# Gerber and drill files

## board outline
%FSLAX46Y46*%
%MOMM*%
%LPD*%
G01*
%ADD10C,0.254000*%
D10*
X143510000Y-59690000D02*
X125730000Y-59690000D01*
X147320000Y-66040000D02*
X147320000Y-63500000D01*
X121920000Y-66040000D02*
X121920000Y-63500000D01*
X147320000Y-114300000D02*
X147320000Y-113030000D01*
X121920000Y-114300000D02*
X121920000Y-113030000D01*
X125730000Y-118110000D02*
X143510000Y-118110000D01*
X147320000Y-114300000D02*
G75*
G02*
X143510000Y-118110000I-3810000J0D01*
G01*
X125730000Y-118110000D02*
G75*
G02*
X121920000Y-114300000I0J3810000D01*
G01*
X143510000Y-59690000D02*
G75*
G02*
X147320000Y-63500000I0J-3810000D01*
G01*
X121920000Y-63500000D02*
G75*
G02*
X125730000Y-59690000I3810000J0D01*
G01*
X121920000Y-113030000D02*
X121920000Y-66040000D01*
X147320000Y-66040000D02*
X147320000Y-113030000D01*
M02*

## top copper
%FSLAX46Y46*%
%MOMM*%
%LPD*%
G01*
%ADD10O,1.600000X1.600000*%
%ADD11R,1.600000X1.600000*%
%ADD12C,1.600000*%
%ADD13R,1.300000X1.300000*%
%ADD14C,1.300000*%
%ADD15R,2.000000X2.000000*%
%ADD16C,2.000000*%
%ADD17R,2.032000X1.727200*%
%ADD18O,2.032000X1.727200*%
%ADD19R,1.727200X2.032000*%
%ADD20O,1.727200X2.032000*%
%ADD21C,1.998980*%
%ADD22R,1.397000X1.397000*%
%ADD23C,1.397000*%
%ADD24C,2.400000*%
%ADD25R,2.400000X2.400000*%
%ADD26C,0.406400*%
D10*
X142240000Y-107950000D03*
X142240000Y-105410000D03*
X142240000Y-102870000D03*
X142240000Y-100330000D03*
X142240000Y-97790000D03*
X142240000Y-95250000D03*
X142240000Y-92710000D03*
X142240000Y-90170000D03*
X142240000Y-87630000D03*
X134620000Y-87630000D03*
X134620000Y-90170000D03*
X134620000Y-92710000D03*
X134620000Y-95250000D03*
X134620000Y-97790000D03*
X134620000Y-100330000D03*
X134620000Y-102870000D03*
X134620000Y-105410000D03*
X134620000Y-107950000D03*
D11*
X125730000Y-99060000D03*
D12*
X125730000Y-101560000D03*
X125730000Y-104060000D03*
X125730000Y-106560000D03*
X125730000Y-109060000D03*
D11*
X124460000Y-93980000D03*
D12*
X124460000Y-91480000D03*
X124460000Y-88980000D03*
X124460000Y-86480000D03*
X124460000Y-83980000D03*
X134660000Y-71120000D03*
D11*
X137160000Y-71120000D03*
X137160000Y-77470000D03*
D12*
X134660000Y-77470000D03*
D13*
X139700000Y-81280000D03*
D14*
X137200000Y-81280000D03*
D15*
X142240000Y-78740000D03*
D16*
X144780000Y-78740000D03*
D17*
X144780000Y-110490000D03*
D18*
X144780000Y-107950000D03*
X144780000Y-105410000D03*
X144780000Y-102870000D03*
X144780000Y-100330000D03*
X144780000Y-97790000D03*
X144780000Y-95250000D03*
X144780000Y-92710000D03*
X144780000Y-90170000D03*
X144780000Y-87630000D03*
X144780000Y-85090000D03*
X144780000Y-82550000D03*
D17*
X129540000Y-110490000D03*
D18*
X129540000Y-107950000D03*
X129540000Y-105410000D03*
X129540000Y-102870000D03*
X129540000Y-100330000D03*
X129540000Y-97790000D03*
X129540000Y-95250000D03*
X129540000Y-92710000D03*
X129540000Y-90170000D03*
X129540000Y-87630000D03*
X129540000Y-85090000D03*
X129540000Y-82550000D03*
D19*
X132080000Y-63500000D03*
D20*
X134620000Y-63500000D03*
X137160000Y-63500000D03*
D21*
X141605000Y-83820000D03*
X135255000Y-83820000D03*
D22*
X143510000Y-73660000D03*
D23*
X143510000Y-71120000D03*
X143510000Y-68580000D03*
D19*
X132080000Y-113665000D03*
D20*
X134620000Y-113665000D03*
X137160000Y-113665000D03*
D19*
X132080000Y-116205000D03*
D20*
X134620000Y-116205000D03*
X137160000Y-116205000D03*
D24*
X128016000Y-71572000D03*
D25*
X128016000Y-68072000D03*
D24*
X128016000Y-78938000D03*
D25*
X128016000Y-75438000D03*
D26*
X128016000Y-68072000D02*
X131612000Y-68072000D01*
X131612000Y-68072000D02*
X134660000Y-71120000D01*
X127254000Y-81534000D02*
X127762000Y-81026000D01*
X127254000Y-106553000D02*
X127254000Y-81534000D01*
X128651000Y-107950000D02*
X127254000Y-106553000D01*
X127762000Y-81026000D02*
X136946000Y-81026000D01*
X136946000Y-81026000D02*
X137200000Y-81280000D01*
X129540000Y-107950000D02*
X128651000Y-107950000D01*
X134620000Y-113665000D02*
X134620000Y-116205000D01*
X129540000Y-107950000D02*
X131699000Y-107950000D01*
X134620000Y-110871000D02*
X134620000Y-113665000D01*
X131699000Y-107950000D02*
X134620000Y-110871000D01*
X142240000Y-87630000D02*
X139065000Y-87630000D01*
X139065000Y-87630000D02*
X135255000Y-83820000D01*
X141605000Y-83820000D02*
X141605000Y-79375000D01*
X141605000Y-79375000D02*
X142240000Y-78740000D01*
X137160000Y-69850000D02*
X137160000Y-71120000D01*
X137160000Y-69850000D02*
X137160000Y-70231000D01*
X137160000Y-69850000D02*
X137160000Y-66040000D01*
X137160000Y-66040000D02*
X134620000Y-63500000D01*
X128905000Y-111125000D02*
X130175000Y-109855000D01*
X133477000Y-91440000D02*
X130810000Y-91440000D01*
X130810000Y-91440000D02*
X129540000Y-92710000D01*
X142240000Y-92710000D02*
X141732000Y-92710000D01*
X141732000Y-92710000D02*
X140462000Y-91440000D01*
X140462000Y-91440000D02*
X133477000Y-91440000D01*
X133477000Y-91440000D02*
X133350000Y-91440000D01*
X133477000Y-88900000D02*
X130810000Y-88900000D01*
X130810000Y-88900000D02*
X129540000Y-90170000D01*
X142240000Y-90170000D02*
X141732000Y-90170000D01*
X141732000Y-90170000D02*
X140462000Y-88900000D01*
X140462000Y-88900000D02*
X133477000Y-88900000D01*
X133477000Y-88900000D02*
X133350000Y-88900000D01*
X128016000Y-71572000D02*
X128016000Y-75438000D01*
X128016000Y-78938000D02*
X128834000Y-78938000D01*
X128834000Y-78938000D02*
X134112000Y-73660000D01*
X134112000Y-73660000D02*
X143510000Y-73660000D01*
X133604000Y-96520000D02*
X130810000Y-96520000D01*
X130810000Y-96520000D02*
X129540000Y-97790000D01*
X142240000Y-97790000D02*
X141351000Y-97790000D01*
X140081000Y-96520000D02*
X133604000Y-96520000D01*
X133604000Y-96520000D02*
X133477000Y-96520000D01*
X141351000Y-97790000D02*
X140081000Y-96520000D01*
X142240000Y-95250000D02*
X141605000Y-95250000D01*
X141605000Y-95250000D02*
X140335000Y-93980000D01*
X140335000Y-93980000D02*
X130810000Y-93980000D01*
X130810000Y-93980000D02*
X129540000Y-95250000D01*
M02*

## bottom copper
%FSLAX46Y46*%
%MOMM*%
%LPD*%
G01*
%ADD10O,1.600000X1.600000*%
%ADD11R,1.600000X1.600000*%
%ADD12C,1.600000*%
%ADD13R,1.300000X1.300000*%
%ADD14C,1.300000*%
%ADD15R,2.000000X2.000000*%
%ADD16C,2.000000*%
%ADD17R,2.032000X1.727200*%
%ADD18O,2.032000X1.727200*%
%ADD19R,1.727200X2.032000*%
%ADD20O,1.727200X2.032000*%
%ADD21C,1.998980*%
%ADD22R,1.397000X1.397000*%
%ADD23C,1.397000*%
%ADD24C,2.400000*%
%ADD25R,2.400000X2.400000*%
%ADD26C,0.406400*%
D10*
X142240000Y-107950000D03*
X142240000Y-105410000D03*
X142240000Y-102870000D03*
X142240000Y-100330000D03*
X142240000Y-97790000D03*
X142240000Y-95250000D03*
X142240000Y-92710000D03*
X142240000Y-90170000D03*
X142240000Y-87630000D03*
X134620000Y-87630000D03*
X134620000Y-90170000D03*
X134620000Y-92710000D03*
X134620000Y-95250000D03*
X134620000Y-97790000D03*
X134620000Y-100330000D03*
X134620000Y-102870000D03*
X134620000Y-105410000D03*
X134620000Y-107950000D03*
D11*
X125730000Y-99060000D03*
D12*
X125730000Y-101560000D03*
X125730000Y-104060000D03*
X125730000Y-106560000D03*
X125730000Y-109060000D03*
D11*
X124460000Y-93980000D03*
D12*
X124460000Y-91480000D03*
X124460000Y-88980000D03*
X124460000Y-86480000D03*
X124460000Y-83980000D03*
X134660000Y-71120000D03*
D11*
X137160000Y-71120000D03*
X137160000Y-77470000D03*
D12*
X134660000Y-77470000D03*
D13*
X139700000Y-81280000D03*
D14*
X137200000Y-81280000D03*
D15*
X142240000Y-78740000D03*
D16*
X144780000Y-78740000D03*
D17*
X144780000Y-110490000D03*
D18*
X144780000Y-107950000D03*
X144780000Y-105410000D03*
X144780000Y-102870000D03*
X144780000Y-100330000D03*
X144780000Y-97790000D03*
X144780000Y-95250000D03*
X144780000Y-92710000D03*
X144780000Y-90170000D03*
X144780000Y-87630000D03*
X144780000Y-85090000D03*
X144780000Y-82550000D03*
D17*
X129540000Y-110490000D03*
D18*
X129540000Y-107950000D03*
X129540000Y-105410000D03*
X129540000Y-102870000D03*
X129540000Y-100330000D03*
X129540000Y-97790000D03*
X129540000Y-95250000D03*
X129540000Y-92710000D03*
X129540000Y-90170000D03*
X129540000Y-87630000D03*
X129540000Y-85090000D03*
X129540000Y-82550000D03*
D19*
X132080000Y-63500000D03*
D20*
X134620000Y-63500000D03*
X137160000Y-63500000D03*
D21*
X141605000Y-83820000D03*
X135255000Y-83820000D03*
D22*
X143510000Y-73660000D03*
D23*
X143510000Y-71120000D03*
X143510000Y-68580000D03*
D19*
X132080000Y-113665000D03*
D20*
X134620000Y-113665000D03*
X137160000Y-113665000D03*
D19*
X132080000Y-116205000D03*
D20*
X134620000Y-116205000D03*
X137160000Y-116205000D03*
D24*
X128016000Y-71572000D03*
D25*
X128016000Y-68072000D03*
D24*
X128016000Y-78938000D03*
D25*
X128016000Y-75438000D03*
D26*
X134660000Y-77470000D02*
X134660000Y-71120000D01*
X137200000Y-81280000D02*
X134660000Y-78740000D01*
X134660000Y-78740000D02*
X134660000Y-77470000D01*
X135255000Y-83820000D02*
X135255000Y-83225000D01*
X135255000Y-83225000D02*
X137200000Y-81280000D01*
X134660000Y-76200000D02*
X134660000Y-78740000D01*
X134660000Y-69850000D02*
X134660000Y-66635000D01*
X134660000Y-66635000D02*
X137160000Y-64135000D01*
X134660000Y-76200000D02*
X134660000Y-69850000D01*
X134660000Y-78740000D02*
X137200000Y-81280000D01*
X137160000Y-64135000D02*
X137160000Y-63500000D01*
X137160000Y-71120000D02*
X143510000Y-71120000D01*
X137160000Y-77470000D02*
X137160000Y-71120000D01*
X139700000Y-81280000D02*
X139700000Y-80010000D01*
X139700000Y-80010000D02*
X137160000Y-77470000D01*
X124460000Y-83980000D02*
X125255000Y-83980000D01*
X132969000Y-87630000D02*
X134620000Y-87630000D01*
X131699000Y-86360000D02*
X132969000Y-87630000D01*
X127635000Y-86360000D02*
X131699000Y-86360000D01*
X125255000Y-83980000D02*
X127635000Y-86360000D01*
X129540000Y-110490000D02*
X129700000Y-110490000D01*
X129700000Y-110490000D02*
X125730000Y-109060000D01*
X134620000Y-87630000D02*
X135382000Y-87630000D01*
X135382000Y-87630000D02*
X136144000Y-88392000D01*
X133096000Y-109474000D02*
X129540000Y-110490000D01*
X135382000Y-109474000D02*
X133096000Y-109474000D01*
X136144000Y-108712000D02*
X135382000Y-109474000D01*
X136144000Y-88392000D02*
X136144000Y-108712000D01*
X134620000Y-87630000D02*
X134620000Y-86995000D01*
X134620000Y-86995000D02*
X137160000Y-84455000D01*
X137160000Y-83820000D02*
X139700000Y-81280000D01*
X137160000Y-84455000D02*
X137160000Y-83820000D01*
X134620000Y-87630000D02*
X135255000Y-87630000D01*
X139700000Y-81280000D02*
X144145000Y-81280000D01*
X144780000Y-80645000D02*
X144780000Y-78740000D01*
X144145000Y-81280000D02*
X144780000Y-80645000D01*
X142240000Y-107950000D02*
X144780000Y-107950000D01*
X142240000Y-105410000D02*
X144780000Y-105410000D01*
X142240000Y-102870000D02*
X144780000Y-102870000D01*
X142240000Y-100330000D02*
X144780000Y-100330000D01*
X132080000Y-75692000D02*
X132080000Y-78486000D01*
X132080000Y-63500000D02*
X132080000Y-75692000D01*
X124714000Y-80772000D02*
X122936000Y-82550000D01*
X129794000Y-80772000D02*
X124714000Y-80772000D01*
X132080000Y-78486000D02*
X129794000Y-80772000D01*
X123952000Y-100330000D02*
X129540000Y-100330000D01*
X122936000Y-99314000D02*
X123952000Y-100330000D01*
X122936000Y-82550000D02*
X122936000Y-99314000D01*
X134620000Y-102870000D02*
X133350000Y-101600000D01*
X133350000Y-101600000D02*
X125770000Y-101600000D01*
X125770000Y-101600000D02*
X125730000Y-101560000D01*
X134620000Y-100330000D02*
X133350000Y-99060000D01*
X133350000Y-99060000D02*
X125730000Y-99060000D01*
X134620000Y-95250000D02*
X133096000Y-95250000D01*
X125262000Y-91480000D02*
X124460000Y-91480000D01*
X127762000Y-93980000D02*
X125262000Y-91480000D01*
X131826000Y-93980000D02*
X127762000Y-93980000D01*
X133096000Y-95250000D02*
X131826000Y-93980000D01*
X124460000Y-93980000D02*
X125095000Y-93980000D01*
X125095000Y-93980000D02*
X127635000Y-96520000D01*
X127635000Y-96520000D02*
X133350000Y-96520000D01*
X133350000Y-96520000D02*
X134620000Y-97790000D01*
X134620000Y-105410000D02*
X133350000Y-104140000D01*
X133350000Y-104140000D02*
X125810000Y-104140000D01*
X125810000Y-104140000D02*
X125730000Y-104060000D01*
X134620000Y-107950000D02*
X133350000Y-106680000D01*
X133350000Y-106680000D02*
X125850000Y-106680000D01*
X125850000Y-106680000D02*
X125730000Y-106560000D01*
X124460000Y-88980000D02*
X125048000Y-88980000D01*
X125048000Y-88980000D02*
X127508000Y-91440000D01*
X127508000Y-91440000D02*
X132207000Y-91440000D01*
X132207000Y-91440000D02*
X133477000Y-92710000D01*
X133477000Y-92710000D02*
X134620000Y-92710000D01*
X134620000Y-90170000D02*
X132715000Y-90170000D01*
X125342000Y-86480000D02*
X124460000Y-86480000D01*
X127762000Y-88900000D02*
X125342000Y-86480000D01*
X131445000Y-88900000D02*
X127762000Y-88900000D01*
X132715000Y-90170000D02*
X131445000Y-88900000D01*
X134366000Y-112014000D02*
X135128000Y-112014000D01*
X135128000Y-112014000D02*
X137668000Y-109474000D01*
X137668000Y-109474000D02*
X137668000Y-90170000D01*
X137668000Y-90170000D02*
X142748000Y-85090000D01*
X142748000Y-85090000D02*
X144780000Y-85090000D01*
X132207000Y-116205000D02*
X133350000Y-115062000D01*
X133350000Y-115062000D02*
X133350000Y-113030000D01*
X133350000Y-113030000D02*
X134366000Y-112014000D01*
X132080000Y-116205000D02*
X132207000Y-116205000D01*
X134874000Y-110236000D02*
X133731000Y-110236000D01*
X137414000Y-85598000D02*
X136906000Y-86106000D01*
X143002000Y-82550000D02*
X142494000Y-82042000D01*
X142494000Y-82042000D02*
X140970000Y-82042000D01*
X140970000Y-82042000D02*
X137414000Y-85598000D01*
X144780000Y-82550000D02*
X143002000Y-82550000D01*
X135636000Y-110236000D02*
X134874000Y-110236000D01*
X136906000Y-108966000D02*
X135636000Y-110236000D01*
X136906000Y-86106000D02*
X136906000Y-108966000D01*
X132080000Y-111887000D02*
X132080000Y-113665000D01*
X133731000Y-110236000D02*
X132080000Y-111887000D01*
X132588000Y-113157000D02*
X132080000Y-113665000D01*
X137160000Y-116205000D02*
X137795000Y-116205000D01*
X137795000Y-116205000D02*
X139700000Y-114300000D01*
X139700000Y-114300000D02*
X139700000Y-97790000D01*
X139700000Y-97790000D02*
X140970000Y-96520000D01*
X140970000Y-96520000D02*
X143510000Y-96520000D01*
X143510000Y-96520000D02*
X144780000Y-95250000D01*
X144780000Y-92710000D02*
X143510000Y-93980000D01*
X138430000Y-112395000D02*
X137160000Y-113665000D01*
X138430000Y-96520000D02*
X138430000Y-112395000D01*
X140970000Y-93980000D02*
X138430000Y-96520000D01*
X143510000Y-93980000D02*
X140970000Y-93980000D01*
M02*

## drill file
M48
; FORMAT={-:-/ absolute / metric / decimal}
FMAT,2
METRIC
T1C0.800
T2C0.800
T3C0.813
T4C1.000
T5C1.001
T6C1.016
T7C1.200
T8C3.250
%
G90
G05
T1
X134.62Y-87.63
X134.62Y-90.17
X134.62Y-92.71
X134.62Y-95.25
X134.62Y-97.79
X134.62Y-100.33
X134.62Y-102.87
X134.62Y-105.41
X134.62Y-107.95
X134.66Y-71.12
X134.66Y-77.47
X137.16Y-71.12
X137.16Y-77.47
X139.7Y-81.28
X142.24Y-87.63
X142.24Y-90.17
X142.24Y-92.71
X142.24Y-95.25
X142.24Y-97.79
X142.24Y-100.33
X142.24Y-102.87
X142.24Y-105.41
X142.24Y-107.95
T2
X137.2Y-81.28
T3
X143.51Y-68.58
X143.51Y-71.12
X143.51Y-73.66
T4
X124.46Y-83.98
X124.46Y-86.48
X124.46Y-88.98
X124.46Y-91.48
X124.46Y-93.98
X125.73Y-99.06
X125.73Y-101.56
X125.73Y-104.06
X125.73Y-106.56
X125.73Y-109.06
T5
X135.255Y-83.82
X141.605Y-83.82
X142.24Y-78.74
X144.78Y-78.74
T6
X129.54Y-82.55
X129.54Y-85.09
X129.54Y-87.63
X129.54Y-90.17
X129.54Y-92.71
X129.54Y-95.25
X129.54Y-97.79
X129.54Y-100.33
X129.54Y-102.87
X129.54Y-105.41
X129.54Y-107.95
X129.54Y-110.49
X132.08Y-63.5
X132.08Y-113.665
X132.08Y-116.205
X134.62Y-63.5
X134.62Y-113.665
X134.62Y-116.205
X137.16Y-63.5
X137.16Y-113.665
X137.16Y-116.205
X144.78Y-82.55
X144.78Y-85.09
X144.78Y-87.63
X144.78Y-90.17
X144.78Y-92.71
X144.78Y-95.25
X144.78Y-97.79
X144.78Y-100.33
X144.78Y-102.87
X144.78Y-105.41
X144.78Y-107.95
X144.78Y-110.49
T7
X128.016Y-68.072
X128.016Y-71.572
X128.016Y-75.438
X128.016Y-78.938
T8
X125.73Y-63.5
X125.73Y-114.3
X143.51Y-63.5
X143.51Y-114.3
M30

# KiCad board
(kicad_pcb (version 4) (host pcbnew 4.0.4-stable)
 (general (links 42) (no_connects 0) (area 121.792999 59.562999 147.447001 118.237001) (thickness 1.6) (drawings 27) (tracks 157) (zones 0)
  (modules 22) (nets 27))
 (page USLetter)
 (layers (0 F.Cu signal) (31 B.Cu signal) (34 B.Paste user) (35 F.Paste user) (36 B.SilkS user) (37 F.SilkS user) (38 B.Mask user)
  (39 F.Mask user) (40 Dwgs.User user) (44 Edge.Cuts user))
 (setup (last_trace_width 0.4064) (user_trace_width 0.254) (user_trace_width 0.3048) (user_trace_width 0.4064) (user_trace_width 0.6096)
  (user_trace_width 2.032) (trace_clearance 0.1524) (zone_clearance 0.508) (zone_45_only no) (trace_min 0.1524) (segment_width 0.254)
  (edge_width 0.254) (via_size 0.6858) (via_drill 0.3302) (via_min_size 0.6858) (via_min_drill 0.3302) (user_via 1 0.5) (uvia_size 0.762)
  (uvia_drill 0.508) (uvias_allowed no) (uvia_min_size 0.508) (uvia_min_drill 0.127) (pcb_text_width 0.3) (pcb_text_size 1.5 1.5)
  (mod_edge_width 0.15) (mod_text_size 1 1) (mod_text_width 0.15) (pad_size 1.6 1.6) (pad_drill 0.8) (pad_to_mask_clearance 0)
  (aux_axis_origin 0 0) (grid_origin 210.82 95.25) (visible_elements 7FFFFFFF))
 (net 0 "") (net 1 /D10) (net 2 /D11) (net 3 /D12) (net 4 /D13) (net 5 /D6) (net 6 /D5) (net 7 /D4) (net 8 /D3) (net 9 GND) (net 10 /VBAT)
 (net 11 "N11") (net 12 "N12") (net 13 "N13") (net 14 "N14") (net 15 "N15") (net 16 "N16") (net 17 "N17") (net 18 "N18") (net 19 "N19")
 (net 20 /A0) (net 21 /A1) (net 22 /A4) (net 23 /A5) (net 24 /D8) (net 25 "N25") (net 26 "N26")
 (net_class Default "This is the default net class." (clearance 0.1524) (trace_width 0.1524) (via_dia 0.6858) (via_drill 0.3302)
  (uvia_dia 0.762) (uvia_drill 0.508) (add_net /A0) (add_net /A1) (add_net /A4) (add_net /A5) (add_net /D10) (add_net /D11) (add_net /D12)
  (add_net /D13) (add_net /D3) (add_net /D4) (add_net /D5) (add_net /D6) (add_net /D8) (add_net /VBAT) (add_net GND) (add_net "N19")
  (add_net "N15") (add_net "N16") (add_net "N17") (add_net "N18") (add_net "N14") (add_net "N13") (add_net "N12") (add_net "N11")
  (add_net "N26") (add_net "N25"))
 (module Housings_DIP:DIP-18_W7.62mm (layer F.Cu) (at 142.24 107.95 180)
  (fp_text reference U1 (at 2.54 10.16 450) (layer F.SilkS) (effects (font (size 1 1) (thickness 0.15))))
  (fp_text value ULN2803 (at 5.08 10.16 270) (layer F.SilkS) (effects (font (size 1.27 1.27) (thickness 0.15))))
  (pad 1 thru_hole oval (at 0 0 180) (size 1.6 1.6) (drill 0.8) (layers *.Cu *.Mask F.SilkS) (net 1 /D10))
  (pad 2 thru_hole oval (at 0 2.54 180) (size 1.6 1.6) (drill 0.8) (layers *.Cu *.Mask F.SilkS) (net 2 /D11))
  (pad 3 thru_hole oval (at 0 5.08 180) (size 1.6 1.6) (drill 0.8) (layers *.Cu *.Mask F.SilkS) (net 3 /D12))
  (pad 4 thru_hole oval (at 0 7.62 180) (size 1.6 1.6) (drill 0.8) (layers *.Cu *.Mask F.SilkS) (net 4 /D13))
  (pad 5 thru_hole oval (at 0 10.16 180) (size 1.6 1.6) (drill 0.8) (layers *.Cu *.Mask F.SilkS) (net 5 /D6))
  (pad 6 thru_hole oval (at 0 12.7 180) (size 1.6 1.6) (drill 0.8) (layers *.Cu *.Mask F.SilkS) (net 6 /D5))
  (pad 7 thru_hole oval (at 0 15.24 180) (size 1.6 1.6) (drill 0.8) (layers *.Cu *.Mask F.SilkS) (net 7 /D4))
  (pad 8 thru_hole oval (at 0 17.78 180) (size 1.6 1.6) (drill 0.8) (layers *.Cu *.Mask F.SilkS) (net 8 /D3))
  (pad 9 thru_hole oval (at 0 20.32 180) (size 1.6 1.6) (drill 0.8) (layers *.Cu *.Mask F.SilkS) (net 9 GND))
  (pad 10 thru_hole oval (at 7.62 20.32 180) (size 1.6 1.6) (drill 0.8) (layers *.Cu *.Mask F.SilkS) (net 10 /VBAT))
  (pad 11 thru_hole oval (at 7.62 17.78 180) (size 1.6 1.6) (drill 0.8) (layers *.Cu *.Mask F.SilkS) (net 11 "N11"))
  (pad 12 thru_hole oval (at 7.62 15.24 180) (size 1.6 1.6) (drill 0.8) (layers *.Cu *.Mask F.SilkS) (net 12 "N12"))
  (pad 13 thru_hole oval (at 7.62 12.7 180) (size 1.6 1.6) (drill 0.8) (layers *.Cu *.Mask F.SilkS) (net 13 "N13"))
  (pad 14 thru_hole oval (at 7.62 10.16 180) (size 1.6 1.6) (drill 0.8) (layers *.Cu *.Mask F.SilkS) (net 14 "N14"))
  (pad 15 thru_hole oval (at 7.62 7.62 180) (size 1.6 1.6) (drill 0.8) (layers *.Cu *.Mask F.SilkS) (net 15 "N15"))
  (pad 16 thru_hole oval (at 7.62 5.08 180) (size 1.6 1.6) (drill 0.8) (layers *.Cu *.Mask F.SilkS) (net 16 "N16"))
  (pad 17 thru_hole oval (at 7.62 2.54 180) (size 1.6 1.6) (drill 0.8) (layers *.Cu *.Mask F.SilkS) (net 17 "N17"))
  (pad 18 thru_hole oval (at 7.62 0 180) (size 1.6 1.6) (drill 0.8) (layers *.Cu *.Mask F.SilkS) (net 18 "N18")))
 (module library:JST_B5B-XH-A (layer F.Cu) (at 125.73 99.06 270)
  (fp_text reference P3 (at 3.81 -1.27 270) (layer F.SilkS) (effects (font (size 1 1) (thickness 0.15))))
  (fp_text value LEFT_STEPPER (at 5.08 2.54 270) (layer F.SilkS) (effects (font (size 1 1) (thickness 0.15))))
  (pad 1 thru_hole rect (at 0 0 270) (size 1.6 1.6) (drill 1) (layers *.Cu *.Mask F.SilkS) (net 15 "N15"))
  (pad 2 thru_hole circle (at 2.5 0 270) (size 1.6 1.6) (drill 1) (layers *.Cu *.Mask F.SilkS) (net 16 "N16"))
  (pad 3 thru_hole circle (at 5 0 270) (size 1.6 1.6) (drill 1) (layers *.Cu *.Mask F.SilkS) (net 17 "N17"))
  (pad 4 thru_hole circle (at 7.5 0 270) (size 1.6 1.6) (drill 1) (layers *.Cu *.Mask F.SilkS) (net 18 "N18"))
  (pad 5 thru_hole circle (at 10 0 270) (size 1.6 1.6) (drill 1) (layers *.Cu *.Mask F.SilkS) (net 10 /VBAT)))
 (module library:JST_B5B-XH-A (layer F.Cu) (at 124.46 93.98 90)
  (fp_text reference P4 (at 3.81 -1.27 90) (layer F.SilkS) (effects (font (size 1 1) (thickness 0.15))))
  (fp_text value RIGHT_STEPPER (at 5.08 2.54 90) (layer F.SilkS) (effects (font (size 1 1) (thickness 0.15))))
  (pad 1 thru_hole rect (at 0 0 90) (size 1.6 1.6) (drill 1) (layers *.Cu *.Mask F.SilkS) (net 14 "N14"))
  (pad 2 thru_hole circle (at 2.5 0 90) (size 1.6 1.6) (drill 1) (layers *.Cu *.Mask F.SilkS) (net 13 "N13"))
  (pad 3 thru_hole circle (at 5 0 90) (size 1.6 1.6) (drill 1) (layers *.Cu *.Mask F.SilkS) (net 12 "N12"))
  (pad 4 thru_hole circle (at 7.5 0 90) (size 1.6 1.6) (drill 1) (layers *.Cu *.Mask F.SilkS) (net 11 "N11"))
  (pad 5 thru_hole circle (at 10 0 90) (size 1.6 1.6) (drill 1) (layers *.Cu *.Mask F.SilkS) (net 10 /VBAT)))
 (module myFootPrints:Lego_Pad (layer F.Cu) (at 125.73 114.3)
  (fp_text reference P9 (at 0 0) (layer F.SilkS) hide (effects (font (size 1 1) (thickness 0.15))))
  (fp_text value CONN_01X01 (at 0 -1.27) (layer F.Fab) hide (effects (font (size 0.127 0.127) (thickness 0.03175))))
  (pad "" np_thru_hole circle (at 0 0) (size 3.25 3.25) (drill 3.25) (layers *.Cu *.Mask)))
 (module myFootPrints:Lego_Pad (layer F.Cu) (at 143.51 114.3)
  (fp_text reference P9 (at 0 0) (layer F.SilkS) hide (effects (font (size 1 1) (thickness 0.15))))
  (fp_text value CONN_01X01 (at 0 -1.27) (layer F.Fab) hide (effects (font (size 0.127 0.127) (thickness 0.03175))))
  (pad "" np_thru_hole circle (at 0 0) (size 3.25 3.25) (drill 3.25) (layers *.Cu *.Mask)))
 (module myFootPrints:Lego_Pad (layer F.Cu) (at 143.51 63.5)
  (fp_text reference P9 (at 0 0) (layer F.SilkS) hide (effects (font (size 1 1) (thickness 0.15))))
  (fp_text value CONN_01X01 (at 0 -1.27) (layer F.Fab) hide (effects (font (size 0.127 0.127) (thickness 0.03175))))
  (pad "" np_thru_hole circle (at 0 0) (size 3.25 3.25) (drill 3.25) (layers *.Cu *.Mask)))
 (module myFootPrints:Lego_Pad (layer F.Cu) (at 125.73 63.5)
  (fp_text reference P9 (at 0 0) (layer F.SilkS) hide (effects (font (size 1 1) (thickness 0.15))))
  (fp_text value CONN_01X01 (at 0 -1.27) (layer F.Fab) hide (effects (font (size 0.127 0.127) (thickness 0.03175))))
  (pad "" np_thru_hole circle (at 0 0) (size 3.25 3.25) (drill 3.25) (layers *.Cu *.Mask)))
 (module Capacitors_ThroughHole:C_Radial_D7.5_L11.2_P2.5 (layer F.Cu) (at 137.16 71.12 180)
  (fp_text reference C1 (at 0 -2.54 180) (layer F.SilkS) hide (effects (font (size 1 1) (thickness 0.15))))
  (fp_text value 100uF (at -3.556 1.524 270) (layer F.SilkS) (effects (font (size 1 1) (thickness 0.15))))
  (pad 2 thru_hole circle (at 2.5 0 180) (size 1.6 1.6) (drill 0.8) (layers *.Cu *.Mask F.SilkS) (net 9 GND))
  (pad 1 thru_hole rect (at 0 0 180) (size 1.6 1.6) (drill 0.8) (layers *.Cu *.Mask F.SilkS) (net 10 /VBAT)))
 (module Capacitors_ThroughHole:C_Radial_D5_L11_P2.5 (layer F.Cu) (at 137.16 77.47 180)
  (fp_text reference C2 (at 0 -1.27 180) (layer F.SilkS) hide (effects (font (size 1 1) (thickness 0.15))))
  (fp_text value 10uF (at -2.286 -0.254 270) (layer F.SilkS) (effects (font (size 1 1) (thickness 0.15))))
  (pad 1 thru_hole rect (at 0 0 180) (size 1.6 1.6) (drill 0.8) (layers *.Cu *.Mask F.SilkS) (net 10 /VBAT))
  (pad 2 thru_hole circle (at 2.5 0 180) (size 1.6 1.6) (drill 0.8) (layers *.Cu *.Mask F.SilkS) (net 9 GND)))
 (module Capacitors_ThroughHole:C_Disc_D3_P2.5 (layer F.Cu) (at 139.7 81.28 180)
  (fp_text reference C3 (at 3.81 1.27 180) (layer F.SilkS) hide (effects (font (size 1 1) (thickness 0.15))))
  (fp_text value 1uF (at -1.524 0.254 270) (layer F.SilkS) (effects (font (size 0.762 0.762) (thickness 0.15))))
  (pad 1 thru_hole rect (at 0 0 180) (size 1.3 1.3) (drill 0.8) (layers *.Cu *.Mask F.SilkS) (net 10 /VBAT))
  (pad 2 thru_hole circle (at 2.5 0 180) (size 1.3 1.3) (drill 0.8001) (layers *.Cu *.Mask F.SilkS) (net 9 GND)))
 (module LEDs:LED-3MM (layer F.Cu) (at 142.24 78.74)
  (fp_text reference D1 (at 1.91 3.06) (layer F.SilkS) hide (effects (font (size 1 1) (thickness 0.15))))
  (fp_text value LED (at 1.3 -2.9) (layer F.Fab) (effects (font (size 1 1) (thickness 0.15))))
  (pad 1 thru_hole rect (at 0 0 90) (size 2 2) (drill 1.00076) (layers *.Cu *.Mask F.SilkS) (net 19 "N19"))
  (pad 2 thru_hole circle (at 2.54 0) (size 2 2) (drill 1.00076) (layers *.Cu *.Mask F.SilkS) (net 10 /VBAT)))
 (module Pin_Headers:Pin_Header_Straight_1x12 (layer F.Cu) (at 144.78 110.49 180)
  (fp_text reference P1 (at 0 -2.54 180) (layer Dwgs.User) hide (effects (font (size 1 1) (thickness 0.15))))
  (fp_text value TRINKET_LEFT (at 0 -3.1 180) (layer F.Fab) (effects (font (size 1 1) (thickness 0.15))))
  (pad 1 thru_hole rect (at 0 0 180) (size 2.032 1.7272) (drill 1.016) (layers *.Cu *.Mask F.SilkS))
  (pad 2 thru_hole oval (at 0 2.54 180) (size 2.032 1.7272) (drill 1.016) (layers *.Cu *.Mask F.SilkS) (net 1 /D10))
  (pad 3 thru_hole oval (at 0 5.08 180) (size 2.032 1.7272) (drill 1.016) (layers *.Cu *.Mask F.SilkS) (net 2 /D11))
  (pad 4 thru_hole oval (at 0 7.62 180) (size 2.032 1.7272) (drill 1.016) (layers *.Cu *.Mask F.SilkS) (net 3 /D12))
  (pad 5 thru_hole oval (at 0 10.16 180) (size 2.032 1.7272) (drill 1.016) (layers *.Cu *.Mask F.SilkS) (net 4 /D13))
  (pad 6 thru_hole oval (at 0 12.7 180) (size 2.032 1.7272) (drill 1.016) (layers *.Cu *.Mask F.SilkS))
  (pad 7 thru_hole oval (at 0 15.24 180) (size 2.032 1.7272) (drill 1.016) (layers *.Cu *.Mask F.SilkS) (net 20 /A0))
  (pad 8 thru_hole oval (at 0 17.78 180) (size 2.032 1.7272) (drill 1.016) (layers *.Cu *.Mask F.SilkS) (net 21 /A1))
  (pad 9 thru_hole oval (at 0 20.32 180) (size 2.032 1.7272) (drill 1.016) (layers *.Cu *.Mask F.SilkS))
  (pad 10 thru_hole oval (at 0 22.86 180) (size 2.032 1.7272) (drill 1.016) (layers *.Cu *.Mask F.SilkS))
  (pad 11 thru_hole oval (at 0 25.4 180) (size 2.032 1.7272) (drill 1.016) (layers *.Cu *.Mask F.SilkS) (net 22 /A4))
  (pad 12 thru_hole oval (at 0 27.94 180) (size 2.032 1.7272) (drill 1.016) (layers *.Cu *.Mask F.SilkS) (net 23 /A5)))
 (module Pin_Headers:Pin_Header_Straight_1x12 (layer F.Cu) (at 129.54 110.49 180)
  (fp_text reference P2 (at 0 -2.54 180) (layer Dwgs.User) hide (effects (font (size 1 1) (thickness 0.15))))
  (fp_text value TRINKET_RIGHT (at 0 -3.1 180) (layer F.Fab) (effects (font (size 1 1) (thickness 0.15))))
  (pad 1 thru_hole rect (at 0 0 180) (size 2.032 1.7272) (drill 1.016) (layers *.Cu *.Mask F.SilkS) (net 10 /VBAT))
  (pad 2 thru_hole oval (at 0 2.54 180) (size 2.032 1.7272) (drill 1.016) (layers *.Cu *.Mask F.SilkS) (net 9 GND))
  (pad 3 thru_hole oval (at 0 5.08 180) (size 2.032 1.7272) (drill 1.016) (layers *.Cu *.Mask F.SilkS))
  (pad 4 thru_hole oval (at 0 7.62 180) (size 2.032 1.7272) (drill 1.016) (layers *.Cu *.Mask F.SilkS))
  (pad 5 thru_hole oval (at 0 10.16 180) (size 2.032 1.7272) (drill 1.016) (layers *.Cu *.Mask F.SilkS) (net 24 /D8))
  (pad 6 thru_hole oval (at 0 12.7 180) (size 2.032 1.7272) (drill 1.016) (layers *.Cu *.Mask F.SilkS) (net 5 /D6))
  (pad 7 thru_hole oval (at 0 15.24 180) (size 2.032 1.7272) (drill 1.016) (layers *.Cu *.Mask F.SilkS) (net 6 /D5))
  (pad 8 thru_hole oval (at 0 17.78 180) (size 2.032 1.7272) (drill 1.016) (layers *.Cu *.Mask F.SilkS) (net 7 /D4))
  (pad 9 thru_hole oval (at 0 20.32 180) (size 2.032 1.7272) (drill 1.016) (layers *.Cu *.Mask F.SilkS) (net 8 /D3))
  (pad 10 thru_hole oval (at 0 22.86 180) (size 2.032 1.7272) (drill 1.016) (layers *.Cu *.Mask F.SilkS))
  (pad 11 thru_hole oval (at 0 25.4 180) (size 2.032 1.7272) (drill 1.016) (layers *.Cu *.Mask F.SilkS))
  (pad 12 thru_hole oval (at 0 27.94 180) (size 2.032 1.7272) (drill 1.016) (layers *.Cu *.Mask F.SilkS)))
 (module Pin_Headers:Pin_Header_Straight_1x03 (layer F.Cu) (at 132.08 63.5 90)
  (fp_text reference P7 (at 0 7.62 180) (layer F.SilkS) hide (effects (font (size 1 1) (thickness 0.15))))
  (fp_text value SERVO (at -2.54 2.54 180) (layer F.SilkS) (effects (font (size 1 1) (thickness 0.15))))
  (pad 1 thru_hole rect (at 0 0 90) (size 2.032 1.7272) (drill 1.016) (layers *.Cu *.Mask F.SilkS) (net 24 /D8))
  (pad 2 thru_hole oval (at 0 2.54 90) (size 2.032 1.7272) (drill 1.016) (layers *.Cu *.Mask F.SilkS) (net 10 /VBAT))
  (pad 3 thru_hole oval (at 0 5.08 90) (size 2.032 1.7272) (drill 1.016) (layers *.Cu *.Mask F.SilkS) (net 9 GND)))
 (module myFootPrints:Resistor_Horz (layer F.Cu) (at 138.43 83.82 180)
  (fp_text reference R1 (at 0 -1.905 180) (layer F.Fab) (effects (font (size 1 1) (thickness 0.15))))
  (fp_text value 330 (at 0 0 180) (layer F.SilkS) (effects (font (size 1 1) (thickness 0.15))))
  (pad 1 thru_hole circle (at -3.175 0 180) (size 1.99898 1.99898) (drill 1.00076) (layers *.Cu *.SilkS *.Mask) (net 19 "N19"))
  (pad 2 thru_hole circle (at 3.175 0 180) (size 1.99898 1.99898) (drill 1.00076) (layers *.Cu *.SilkS *.Mask) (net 9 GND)))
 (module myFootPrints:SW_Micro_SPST (layer F.Cu) (at 143.51 71.12 90)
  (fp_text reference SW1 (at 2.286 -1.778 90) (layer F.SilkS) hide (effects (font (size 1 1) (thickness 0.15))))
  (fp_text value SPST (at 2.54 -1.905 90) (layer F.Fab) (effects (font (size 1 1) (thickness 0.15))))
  (pad 1 thru_hole rect (at -2.54 0 90) (size 1.397 1.397) (drill 0.8128) (layers *.Cu *.Mask F.SilkS) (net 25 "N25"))
  (pad 2 thru_hole circle (at 0 0 90) (size 1.397 1.397) (drill 0.8128) (layers *.Cu *.Mask F.SilkS) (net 10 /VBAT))
  (pad 3 thru_hole circle (at 2.54 0 90) (size 1.397 1.397) (drill 0.8128) (layers *.Cu *.Mask F.SilkS)))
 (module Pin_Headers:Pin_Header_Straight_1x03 (layer F.Cu) (at 132.08 113.665 90)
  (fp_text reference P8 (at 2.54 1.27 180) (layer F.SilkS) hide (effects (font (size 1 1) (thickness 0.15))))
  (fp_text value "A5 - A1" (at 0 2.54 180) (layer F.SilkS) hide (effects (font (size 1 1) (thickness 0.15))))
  (pad 1 thru_hole rect (at 0 0 90) (size 2.032 1.7272) (drill 1.016) (layers *.Cu *.Mask F.SilkS) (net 23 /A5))
  (pad 2 thru_hole oval (at 0 2.54 90) (size 2.032 1.7272) (drill 1.016) (layers *.Cu *.Mask F.SilkS) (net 9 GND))
  (pad 3 thru_hole oval (at 0 5.08 90) (size 2.032 1.7272) (drill 1.016) (layers *.Cu *.Mask F.SilkS) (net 21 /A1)))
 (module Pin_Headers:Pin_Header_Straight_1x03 (layer F.Cu) (at 132.08 116.205 90)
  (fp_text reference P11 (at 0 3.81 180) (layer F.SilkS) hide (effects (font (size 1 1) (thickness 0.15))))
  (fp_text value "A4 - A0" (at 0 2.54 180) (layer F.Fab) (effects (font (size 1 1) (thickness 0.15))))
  (pad 1 thru_hole rect (at 0 0 90) (size 2.032 1.7272) (drill 1.016) (layers *.Cu *.Mask F.SilkS) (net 22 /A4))
  (pad 2 thru_hole oval (at 0 2.54 90) (size 2.032 1.7272) (drill 1.016) (layers *.Cu *.Mask F.SilkS) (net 9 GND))
  (pad 3 thru_hole oval (at 0 5.08 90) (size 2.032 1.7272) (drill 1.016) (layers *.Cu *.Mask F.SilkS) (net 20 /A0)))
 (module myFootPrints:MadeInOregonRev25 (layer F.Cu) (at 138.43 102.235 90)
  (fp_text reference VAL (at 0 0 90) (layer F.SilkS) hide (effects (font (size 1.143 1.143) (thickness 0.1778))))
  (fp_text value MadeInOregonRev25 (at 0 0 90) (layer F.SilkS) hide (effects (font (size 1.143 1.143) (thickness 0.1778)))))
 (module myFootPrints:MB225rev (layer F.Cu) (at 138.43 109.22 90)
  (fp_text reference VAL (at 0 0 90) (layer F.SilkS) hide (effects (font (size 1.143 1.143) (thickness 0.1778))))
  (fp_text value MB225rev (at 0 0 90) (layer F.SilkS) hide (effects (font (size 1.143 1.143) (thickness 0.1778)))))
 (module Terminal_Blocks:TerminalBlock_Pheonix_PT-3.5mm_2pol (layer F.Cu) (at 128.016 68.072 270)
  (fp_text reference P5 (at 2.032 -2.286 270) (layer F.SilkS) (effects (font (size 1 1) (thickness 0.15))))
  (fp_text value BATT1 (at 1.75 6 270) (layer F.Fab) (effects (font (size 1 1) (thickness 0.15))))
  (pad 2 thru_hole circle (at 3.5 0 270) (size 2.4 2.4) (drill 1.2) (layers *.Cu *.Mask F.SilkS) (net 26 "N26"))
  (pad 1 thru_hole rect (at 0 0 270) (size 2.4 2.4) (drill 1.2) (layers *.Cu *.Mask F.SilkS) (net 9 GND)))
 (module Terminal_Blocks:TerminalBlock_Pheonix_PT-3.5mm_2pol (layer F.Cu) (at 128.016 75.438 270)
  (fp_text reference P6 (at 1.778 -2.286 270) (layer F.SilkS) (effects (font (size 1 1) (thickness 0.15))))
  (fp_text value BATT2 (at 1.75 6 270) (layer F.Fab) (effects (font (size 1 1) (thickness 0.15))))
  (pad 2 thru_hole circle (at 3.5 0 270) (size 2.4 2.4) (drill 1.2) (layers *.Cu *.Mask F.SilkS) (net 25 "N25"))
  (pad 1 thru_hole rect (at 0 0 270) (size 2.4 2.4) (drill 1.2) (layers *.Cu *.Mask F.SilkS) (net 26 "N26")))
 (gr_line (start 143.51 59.69) (end 125.73 59.69) (angle 90) (layer Edge.Cuts) (width 0.254))
 (gr_line (start 147.32 66.04) (end 147.32 63.5) (angle 90) (layer Edge.Cuts) (width 0.254))
 (gr_line (start 121.92 66.04) (end 121.92 63.5) (angle 90) (layer Edge.Cuts) (width 0.254))
 (gr_line (start 147.32 114.3) (end 147.32 113.03) (angle 90) (layer Edge.Cuts) (width 0.254))
 (gr_line (start 121.92 114.3) (end 121.92 113.03) (angle 90) (layer Edge.Cuts) (width 0.254))
 (gr_line (start 125.73 118.11) (end 143.51 118.11) (angle 90) (layer Edge.Cuts) (width 0.254))
 (gr_arc (start 143.51 114.3) (end 147.32 114.3) (angle 90) (layer Edge.Cuts) (width 0.254))
 (gr_arc (start 125.73 114.3) (end 125.73 118.11) (angle 90) (layer Edge.Cuts) (width 0.254))
 (gr_arc (start 143.51 63.5) (end 143.51 59.69) (angle 90) (layer Edge.Cuts) (width 0.254))
 (gr_arc (start 125.73 63.5) (end 121.92 63.5) (angle 90) (layer Edge.Cuts) (width 0.254))
 (gr_line (start 121.92 113.03) (end 121.92 66.04) (angle 90) (layer Edge.Cuts) (width 0.254))
 (gr_line (start 147.32 66.04) (end 147.32 113.03) (angle 90) (layer Edge.Cuts) (width 0.254))
 (segment (start 134.66 77.47) (end 134.66 71.12) (width 0.4064) (layer B.Cu) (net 9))
 (segment (start 137.2 81.28) (end 134.66 78.74) (width 0.4064) (layer B.Cu) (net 9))
 (segment (start 134.66 78.74) (end 134.66 77.47) (width 0.4064) (layer B.Cu) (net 9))
 (segment (start 128.016 68.072) (end 131.612 68.072) (width 0.4064) (layer F.Cu) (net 9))
 (segment (start 131.612 68.072) (end 134.66 71.12) (width 0.4064) (layer F.Cu) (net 9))
 (segment (start 127.254 81.534) (end 127.762 81.026) (width 0.4064) (layer F.Cu) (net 9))
 (segment (start 127.254 106.553) (end 127.254 81.534) (width 0.4064) (layer F.Cu) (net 9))
 (segment (start 128.651 107.95) (end 127.254 106.553) (width 0.4064) (layer F.Cu) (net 9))
 (segment (start 127.762 81.026) (end 136.946 81.026) (width 0.4064) (layer F.Cu) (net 9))
 (segment (start 136.946 81.026) (end 137.2 81.28) (width 0.4064) (layer F.Cu) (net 9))
 (segment (start 129.54 107.95) (end 128.651 107.95) (width 0.4064) (layer F.Cu) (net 9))
 (segment (start 134.62 113.665) (end 134.62 116.205) (width 0.4064) (layer F.Cu) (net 9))
 (segment (start 129.54 107.95) (end 131.699 107.95) (width 0.4064) (layer F.Cu) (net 9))
 (segment (start 134.62 110.871) (end 134.62 113.665) (width 0.4064) (layer F.Cu) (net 9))
 (segment (start 131.699 107.95) (end 134.62 110.871) (width 0.4064) (layer F.Cu) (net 9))
 (segment (start 142.24 87.63) (end 139.065 87.63) (width 0.4064) (layer F.Cu) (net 9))
 (segment (start 139.065 87.63) (end 135.255 83.82) (width 0.4064) (layer F.Cu) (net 9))
 (segment (start 135.255 83.82) (end 135.255 83.225) (width 0.4064) (layer B.Cu) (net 9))
 (segment (start 135.255 83.225) (end 137.2 81.28) (width 0.4064) (layer B.Cu) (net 9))
 (segment (start 134.66 76.2) (end 134.66 78.74) (width 0.4064) (layer B.Cu) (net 9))
 (segment (start 134.66 69.85) (end 134.66 66.635) (width 0.4064) (layer B.Cu) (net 9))
 (segment (start 134.66 66.635) (end 137.16 64.135) (width 0.4064) (layer B.Cu) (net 9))
 (segment (start 134.66 76.2) (end 134.66 69.85) (width 0.4064) (layer B.Cu) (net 9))
 (segment (start 134.66 78.74) (end 137.2 81.28) (width 0.4064) (layer B.Cu) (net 9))
 (segment (start 137.16 64.135) (end 137.16 63.5) (width 0.4064) (layer B.Cu) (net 9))
 (segment (start 141.605 83.82) (end 141.605 79.375) (width 0.4064) (layer F.Cu) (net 19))
 (segment (start 141.605 79.375) (end 142.24 78.74) (width 0.4064) (layer F.Cu) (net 19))
 (segment (start 137.16 69.85) (end 137.16 71.12) (width 0.4064) (layer F.Cu) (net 10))
 (segment (start 137.16 71.12) (end 143.51 71.12) (width 0.4064) (layer B.Cu) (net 10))
 (segment (start 137.16 77.47) (end 137.16 71.12) (width 0.4064) (layer B.Cu) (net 10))
 (segment (start 139.7 81.28) (end 139.7 80.01) (width 0.4064) (layer B.Cu) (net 10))
 (segment (start 139.7 80.01) (end 137.16 77.47) (width 0.4064) (layer B.Cu) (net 10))
 (segment (start 124.46 83.98) (end 125.255 83.98) (width 0.4064) (layer B.Cu) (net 10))
 (segment (start 132.969 87.63) (end 134.62 87.63) (width 0.4064) (layer B.Cu) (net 10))
 (segment (start 131.699 86.36) (end 132.969 87.63) (width 0.4064) (layer B.Cu) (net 10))
 (segment (start 127.635 86.36) (end 131.699 86.36) (width 0.4064) (layer B.Cu) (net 10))
 (segment (start 125.255 83.98) (end 127.635 86.36) (width 0.4064) (layer B.Cu) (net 10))
 (segment (start 137.16 69.85) (end 137.16 70.231) (width 0.4064) (layer F.Cu) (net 10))
 (segment (start 137.16 69.85) (end 137.16 66.04) (width 0.4064) (layer F.Cu) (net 10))
 (segment (start 137.16 66.04) (end 134.62 63.5) (width 0.4064) (layer F.Cu) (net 10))
 (segment (start 129.54 110.49) (end 129.7 110.49) (width 0.4064) (layer B.Cu) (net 10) (status 10))
 (segment (start 129.7 110.49) (end 125.73 109.06) (width 0.4064) (layer B.Cu) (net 10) (status 20))
 (segment (start 134.62 87.63) (end 135.382 87.63) (width 0.4064) (layer B.Cu) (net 10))
 (segment (start 135.382 87.63) (end 136.144 88.392) (width 0.4064) (layer B.Cu) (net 10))
 (segment (start 133.096 109.474) (end 129.54 110.49) (width 0.4064) (layer B.Cu) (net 10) (status 20))
 (segment (start 135.382 109.474) (end 133.096 109.474) (width 0.4064) (layer B.Cu) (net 10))
 (segment (start 136.144 108.712) (end 135.382 109.474) (width 0.4064) (layer B.Cu) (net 10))
 (segment (start 136.144 88.392) (end 136.144 108.712) (width 0.4064) (layer B.Cu) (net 10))
 (segment (start 134.62 87.63) (end 134.62 86.995) (width 0.4064) (layer B.Cu) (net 10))
 (segment (start 134.62 86.995) (end 137.16 84.455) (width 0.4064) (layer B.Cu) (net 10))
 (segment (start 137.16 83.82) (end 139.7 81.28) (width 0.4064) (layer B.Cu) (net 10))
 (segment (start 137.16 84.455) (end 137.16 83.82) (width 0.4064) (layer B.Cu) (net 10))
 (segment (start 134.62 87.63) (end 135.255 87.63) (width 0.4064) (layer B.Cu) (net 10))
 (segment (start 139.7 81.28) (end 144.145 81.28) (width 0.4064) (layer B.Cu) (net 10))
 (segment (start 144.78 80.645) (end 144.78 78.74) (width 0.4064) (layer B.Cu) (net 10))
 (segment (start 144.145 81.28) (end 144.78 80.645) (width 0.4064) (layer B.Cu) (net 10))
 (segment (start 128.905 111.125) (end 130.175 109.855) (width 0.4064) (layer F.Cu) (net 10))
 (segment (start 142.24 107.95) (end 144.78 107.95) (width 0.4064) (layer B.Cu) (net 1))
 (segment (start 142.24 105.41) (end 144.78 105.41) (width 0.4064) (layer B.Cu) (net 2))
 (segment (start 142.24 102.87) (end 144.78 102.87) (width 0.4064) (layer B.Cu) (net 3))
 (segment (start 142.24 100.33) (end 144.78 100.33) (width 0.4064) (layer B.Cu) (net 4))
 (segment (start 132.08 75.692) (end 132.08 78.486) (width 0.4064) (layer B.Cu) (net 24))
 (segment (start 132.08 63.5) (end 132.08 75.692) (width 0.4064) (layer B.Cu) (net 24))
 (segment (start 124.714 80.772) (end 122.936 82.55) (width 0.4064) (layer B.Cu) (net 24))
 (segment (start 129.794 80.772) (end 124.714 80.772) (width 0.4064) (layer B.Cu) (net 24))
 (segment (start 132.08 78.486) (end 129.794 80.772) (width 0.4064) (layer B.Cu) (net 24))
 (segment (start 123.952 100.33) (end 129.54 100.33) (width 0.4064) (layer B.Cu) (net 24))
 (segment (start 122.936 99.314) (end 123.952 100.33) (width 0.4064) (layer B.Cu) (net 24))
 (segment (start 122.936 82.55) (end 122.936 99.314) (width 0.4064) (layer B.Cu) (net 24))
 (segment (start 133.477 91.44) (end 130.81 91.44) (width 0.4064) (layer F.Cu) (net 7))
 (segment (start 130.81 91.44) (end 129.54 92.71) (width 0.4064) (layer F.Cu) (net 7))
 (segment (start 142.24 92.71) (end 141.732 92.71) (width 0.4064) (layer F.Cu) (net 7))
 (segment (start 141.732 92.71) (end 140.462 91.44) (width 0.4064) (layer F.Cu) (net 7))
 (segment (start 140.462 91.44) (end 133.477 91.44) (width 0.4064) (layer F.Cu) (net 7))
 (segment (start 133.477 91.44) (end 133.35 91.44) (width 0.4064) (layer F.Cu) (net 7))
 (segment (start 133.477 88.9) (end 130.81 88.9) (width 0.4064) (layer F.Cu) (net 8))
 (segment (start 130.81 88.9) (end 129.54 90.17) (width 0.4064) (layer F.Cu) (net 8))
 (segment (start 142.24 90.17) (end 141.732 90.17) (width 0.4064) (layer F.Cu) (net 8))
 (segment (start 141.732 90.17) (end 140.462 88.9) (width 0.4064) (layer F.Cu) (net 8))
 (segment (start 140.462 88.9) (end 133.477 88.9) (width 0.4064) (layer F.Cu) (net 8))
 (segment (start 133.477 88.9) (end 133.35 88.9) (width 0.4064) (layer F.Cu) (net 8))
 (segment (start 134.62 102.87) (end 133.35 101.6) (width 0.4064) (layer B.Cu) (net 16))
 (segment (start 133.35 101.6) (end 125.77 101.6) (width 0.4064) (layer B.Cu) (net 16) (status 20))
 (segment (start 125.77 101.6) (end 125.73 101.56) (width 0.4064) (layer B.Cu) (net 16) (status 30))
 (segment (start 134.62 100.33) (end 133.35 99.06) (width 0.4064) (layer B.Cu) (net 15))
 (segment (start 133.35 99.06) (end 125.73 99.06) (width 0.4064) (layer B.Cu) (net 15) (status 20))
 (segment (start 134.62 95.25) (end 133.096 95.25) (width 0.4064) (layer B.Cu) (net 13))
 (segment (start 125.262 91.48) (end 124.46 91.48) (width 0.4064) (layer B.Cu) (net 13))
 (segment (start 127.762 93.98) (end 125.262 91.48) (width 0.4064) (layer B.Cu) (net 13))
 (segment (start 131.826 93.98) (end 127.762 93.98) (width 0.4064) (layer B.Cu) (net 13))
 (segment (start 133.096 95.25) (end 131.826 93.98) (width 0.4064) (layer B.Cu) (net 13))
 (segment (start 124.46 93.98) (end 125.095 93.98) (width 0.4064) (layer B.Cu) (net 14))
 (segment (start 125.095 93.98) (end 127.635 96.52) (width 0.4064) (layer B.Cu) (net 14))
 (segment (start 127.635 96.52) (end 133.35 96.52) (width 0.4064) (layer B.Cu) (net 14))
 (segment (start 133.35 96.52) (end 134.62 97.79) (width 0.4064) (layer B.Cu) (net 14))
 (segment (start 128.016 71.572) (end 128.016 75.438) (width 0.4064) (layer F.Cu) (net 26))
 (segment (start 128.016 78.938) (end 128.834 78.938) (width 0.4064) (layer F.Cu) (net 25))
 (segment (start 128.834 78.938) (end 134.112 73.66) (width 0.4064) (layer F.Cu) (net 25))
 (segment (start 134.112 73.66) (end 143.51 73.66) (width 0.4064) (layer F.Cu) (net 25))
 (segment (start 134.62 105.41) (end 133.35 104.14) (width 0.4064) (layer B.Cu) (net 17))
 (segment (start 133.35 104.14) (end 125.81 104.14) (width 0.4064) (layer B.Cu) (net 17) (status 20))
 (segment (start 125.81 104.14) (end 125.73 104.06) (width 0.4064) (layer B.Cu) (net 17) (status 30))
 (segment (start 134.62 107.95) (end 133.35 106.68) (width 0.4064) (layer B.Cu) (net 18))
 (segment (start 133.35 106.68) (end 125.85 106.68) (width 0.4064) (layer B.Cu) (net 18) (status 20))
 (segment (start 125.85 106.68) (end 125.73 106.56) (width 0.4064) (layer B.Cu) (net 18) (status 30))
 (segment (start 124.46 88.98) (end 125.048 88.98) (width 0.4064) (layer B.Cu) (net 12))
 (segment (start 125.048 88.98) (end 127.508 91.44) (width 0.4064) (layer B.Cu) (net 12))
 (segment (start 127.508 91.44) (end 132.207 91.44) (width 0.4064) (layer B.Cu) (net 12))
 (segment (start 132.207 91.44) (end 133.477 92.71) (width 0.4064) (layer B.Cu) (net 12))
 (segment (start 133.477 92.71) (end 134.62 92.71) (width 0.4064) (layer B.Cu) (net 12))
 (segment (start 134.62 90.17) (end 132.715 90.17) (width 0.4064) (layer B.Cu) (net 11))
 (segment (start 125.342 86.48) (end 124.46 86.48) (width 0.4064) (layer B.Cu) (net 11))
 (segment (start 127.762 88.9) (end 125.342 86.48) (width 0.4064) (layer B.Cu) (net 11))
 (segment (start 131.445 88.9) (end 127.762 88.9) (width 0.4064) (layer B.Cu) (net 11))
 (segment (start 132.715 90.17) (end 131.445 88.9) (width 0.4064) (layer B.Cu) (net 11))
 (segment (start 134.366 112.014) (end 135.128 112.014) (width 0.4064) (layer B.Cu) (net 22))
 (segment (start 135.128 112.014) (end 137.668 109.474) (width 0.4064) (layer B.Cu) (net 22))
 (segment (start 137.668 109.474) (end 137.668 90.17) (width 0.4064) (layer B.Cu) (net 22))
 (segment (start 137.668 90.17) (end 142.748 85.09) (width 0.4064) (layer B.Cu) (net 22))
 (segment (start 142.748 85.09) (end 144.78 85.09) (width 0.4064) (layer B.Cu) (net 22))
 (segment (start 132.207 116.205) (end 133.35 115.062) (width 0.4064) (layer B.Cu) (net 22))
 (segment (start 133.35 115.062) (end 133.35 113.03) (width 0.4064) (layer B.Cu) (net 22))
 (segment (start 133.35 113.03) (end 134.366 112.014) (width 0.4064) (layer B.Cu) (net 22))
 (segment (start 132.08 116.205) (end 132.207 116.205) (width 0.4064) (layer B.Cu) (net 22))
 (segment (start 134.874 110.236) (end 133.731 110.236) (width 0.4064) (layer B.Cu) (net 23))
 (segment (start 137.414 85.598) (end 136.906 86.106) (width 0.4064) (layer B.Cu) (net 23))
 (segment (start 143.002 82.55) (end 142.494 82.042) (width 0.4064) (layer B.Cu) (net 23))
 (segment (start 142.494 82.042) (end 140.97 82.042) (width 0.4064) (layer B.Cu) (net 23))
 (segment (start 140.97 82.042) (end 137.414 85.598) (width 0.4064) (layer B.Cu) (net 23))
 (segment (start 144.78 82.55) (end 143.002 82.55) (width 0.4064) (layer B.Cu) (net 23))
 (segment (start 135.636 110.236) (end 134.874 110.236) (width 0.4064) (layer B.Cu) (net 23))
 (segment (start 136.906 108.966) (end 135.636 110.236) (width 0.4064) (layer B.Cu) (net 23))
 (segment (start 136.906 86.106) (end 136.906 108.966) (width 0.4064) (layer B.Cu) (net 23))
 (segment (start 132.08 111.887) (end 132.08 113.665) (width 0.4064) (layer B.Cu) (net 23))
 (segment (start 133.731 110.236) (end 132.08 111.887) (width 0.4064) (layer B.Cu) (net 23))
 (segment (start 132.588 113.157) (end 132.08 113.665) (width 0.4064) (layer B.Cu) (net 23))
 (segment (start 137.16 116.205) (end 137.795 116.205) (width 0.4064) (layer B.Cu) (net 20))
 (segment (start 137.795 116.205) (end 139.7 114.3) (width 0.4064) (layer B.Cu) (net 20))
 (segment (start 139.7 114.3) (end 139.7 97.79) (width 0.4064) (layer B.Cu) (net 20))
 (segment (start 139.7 97.79) (end 140.97 96.52) (width 0.4064) (layer B.Cu) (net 20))
 (segment (start 140.97 96.52) (end 143.51 96.52) (width 0.4064) (layer B.Cu) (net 20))
 (segment (start 143.51 96.52) (end 144.78 95.25) (width 0.4064) (layer B.Cu) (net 20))
 (segment (start 144.78 92.71) (end 143.51 93.98) (width 0.4064) (layer B.Cu) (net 21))
 (segment (start 138.43 112.395) (end 137.16 113.665) (width 0.4064) (layer B.Cu) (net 21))
 (segment (start 138.43 96.52) (end 138.43 112.395) (width 0.4064) (layer B.Cu) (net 21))
 (segment (start 140.97 93.98) (end 138.43 96.52) (width 0.4064) (layer B.Cu) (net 21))
 (segment (start 143.51 93.98) (end 140.97 93.98) (width 0.4064) (layer B.Cu) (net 21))
 (segment (start 133.604 96.52) (end 130.81 96.52) (width 0.4064) (layer F.Cu) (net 5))
 (segment (start 130.81 96.52) (end 129.54 97.79) (width 0.4064) (layer F.Cu) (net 5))
 (segment (start 142.24 97.79) (end 141.351 97.79) (width 0.4064) (layer F.Cu) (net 5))
 (segment (start 140.081 96.52) (end 133.604 96.52) (width 0.4064) (layer F.Cu) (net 5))
 (segment (start 133.604 96.52) (end 133.477 96.52) (width 0.4064) (layer F.Cu) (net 5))
 (segment (start 141.351 97.79) (end 140.081 96.52) (width 0.4064) (layer F.Cu) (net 5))
 (segment (start 142.24 95.25) (end 141.605 95.25) (width 0.4064) (layer F.Cu) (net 6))
 (segment (start 141.605 95.25) (end 140.335 93.98) (width 0.4064) (layer F.Cu) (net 6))
 (segment (start 140.335 93.98) (end 130.81 93.98) (width 0.4064) (layer F.Cu) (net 6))
 (segment (start 130.81 93.98) (end 129.54 95.25) (width 0.4064) (layer F.Cu) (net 6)))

